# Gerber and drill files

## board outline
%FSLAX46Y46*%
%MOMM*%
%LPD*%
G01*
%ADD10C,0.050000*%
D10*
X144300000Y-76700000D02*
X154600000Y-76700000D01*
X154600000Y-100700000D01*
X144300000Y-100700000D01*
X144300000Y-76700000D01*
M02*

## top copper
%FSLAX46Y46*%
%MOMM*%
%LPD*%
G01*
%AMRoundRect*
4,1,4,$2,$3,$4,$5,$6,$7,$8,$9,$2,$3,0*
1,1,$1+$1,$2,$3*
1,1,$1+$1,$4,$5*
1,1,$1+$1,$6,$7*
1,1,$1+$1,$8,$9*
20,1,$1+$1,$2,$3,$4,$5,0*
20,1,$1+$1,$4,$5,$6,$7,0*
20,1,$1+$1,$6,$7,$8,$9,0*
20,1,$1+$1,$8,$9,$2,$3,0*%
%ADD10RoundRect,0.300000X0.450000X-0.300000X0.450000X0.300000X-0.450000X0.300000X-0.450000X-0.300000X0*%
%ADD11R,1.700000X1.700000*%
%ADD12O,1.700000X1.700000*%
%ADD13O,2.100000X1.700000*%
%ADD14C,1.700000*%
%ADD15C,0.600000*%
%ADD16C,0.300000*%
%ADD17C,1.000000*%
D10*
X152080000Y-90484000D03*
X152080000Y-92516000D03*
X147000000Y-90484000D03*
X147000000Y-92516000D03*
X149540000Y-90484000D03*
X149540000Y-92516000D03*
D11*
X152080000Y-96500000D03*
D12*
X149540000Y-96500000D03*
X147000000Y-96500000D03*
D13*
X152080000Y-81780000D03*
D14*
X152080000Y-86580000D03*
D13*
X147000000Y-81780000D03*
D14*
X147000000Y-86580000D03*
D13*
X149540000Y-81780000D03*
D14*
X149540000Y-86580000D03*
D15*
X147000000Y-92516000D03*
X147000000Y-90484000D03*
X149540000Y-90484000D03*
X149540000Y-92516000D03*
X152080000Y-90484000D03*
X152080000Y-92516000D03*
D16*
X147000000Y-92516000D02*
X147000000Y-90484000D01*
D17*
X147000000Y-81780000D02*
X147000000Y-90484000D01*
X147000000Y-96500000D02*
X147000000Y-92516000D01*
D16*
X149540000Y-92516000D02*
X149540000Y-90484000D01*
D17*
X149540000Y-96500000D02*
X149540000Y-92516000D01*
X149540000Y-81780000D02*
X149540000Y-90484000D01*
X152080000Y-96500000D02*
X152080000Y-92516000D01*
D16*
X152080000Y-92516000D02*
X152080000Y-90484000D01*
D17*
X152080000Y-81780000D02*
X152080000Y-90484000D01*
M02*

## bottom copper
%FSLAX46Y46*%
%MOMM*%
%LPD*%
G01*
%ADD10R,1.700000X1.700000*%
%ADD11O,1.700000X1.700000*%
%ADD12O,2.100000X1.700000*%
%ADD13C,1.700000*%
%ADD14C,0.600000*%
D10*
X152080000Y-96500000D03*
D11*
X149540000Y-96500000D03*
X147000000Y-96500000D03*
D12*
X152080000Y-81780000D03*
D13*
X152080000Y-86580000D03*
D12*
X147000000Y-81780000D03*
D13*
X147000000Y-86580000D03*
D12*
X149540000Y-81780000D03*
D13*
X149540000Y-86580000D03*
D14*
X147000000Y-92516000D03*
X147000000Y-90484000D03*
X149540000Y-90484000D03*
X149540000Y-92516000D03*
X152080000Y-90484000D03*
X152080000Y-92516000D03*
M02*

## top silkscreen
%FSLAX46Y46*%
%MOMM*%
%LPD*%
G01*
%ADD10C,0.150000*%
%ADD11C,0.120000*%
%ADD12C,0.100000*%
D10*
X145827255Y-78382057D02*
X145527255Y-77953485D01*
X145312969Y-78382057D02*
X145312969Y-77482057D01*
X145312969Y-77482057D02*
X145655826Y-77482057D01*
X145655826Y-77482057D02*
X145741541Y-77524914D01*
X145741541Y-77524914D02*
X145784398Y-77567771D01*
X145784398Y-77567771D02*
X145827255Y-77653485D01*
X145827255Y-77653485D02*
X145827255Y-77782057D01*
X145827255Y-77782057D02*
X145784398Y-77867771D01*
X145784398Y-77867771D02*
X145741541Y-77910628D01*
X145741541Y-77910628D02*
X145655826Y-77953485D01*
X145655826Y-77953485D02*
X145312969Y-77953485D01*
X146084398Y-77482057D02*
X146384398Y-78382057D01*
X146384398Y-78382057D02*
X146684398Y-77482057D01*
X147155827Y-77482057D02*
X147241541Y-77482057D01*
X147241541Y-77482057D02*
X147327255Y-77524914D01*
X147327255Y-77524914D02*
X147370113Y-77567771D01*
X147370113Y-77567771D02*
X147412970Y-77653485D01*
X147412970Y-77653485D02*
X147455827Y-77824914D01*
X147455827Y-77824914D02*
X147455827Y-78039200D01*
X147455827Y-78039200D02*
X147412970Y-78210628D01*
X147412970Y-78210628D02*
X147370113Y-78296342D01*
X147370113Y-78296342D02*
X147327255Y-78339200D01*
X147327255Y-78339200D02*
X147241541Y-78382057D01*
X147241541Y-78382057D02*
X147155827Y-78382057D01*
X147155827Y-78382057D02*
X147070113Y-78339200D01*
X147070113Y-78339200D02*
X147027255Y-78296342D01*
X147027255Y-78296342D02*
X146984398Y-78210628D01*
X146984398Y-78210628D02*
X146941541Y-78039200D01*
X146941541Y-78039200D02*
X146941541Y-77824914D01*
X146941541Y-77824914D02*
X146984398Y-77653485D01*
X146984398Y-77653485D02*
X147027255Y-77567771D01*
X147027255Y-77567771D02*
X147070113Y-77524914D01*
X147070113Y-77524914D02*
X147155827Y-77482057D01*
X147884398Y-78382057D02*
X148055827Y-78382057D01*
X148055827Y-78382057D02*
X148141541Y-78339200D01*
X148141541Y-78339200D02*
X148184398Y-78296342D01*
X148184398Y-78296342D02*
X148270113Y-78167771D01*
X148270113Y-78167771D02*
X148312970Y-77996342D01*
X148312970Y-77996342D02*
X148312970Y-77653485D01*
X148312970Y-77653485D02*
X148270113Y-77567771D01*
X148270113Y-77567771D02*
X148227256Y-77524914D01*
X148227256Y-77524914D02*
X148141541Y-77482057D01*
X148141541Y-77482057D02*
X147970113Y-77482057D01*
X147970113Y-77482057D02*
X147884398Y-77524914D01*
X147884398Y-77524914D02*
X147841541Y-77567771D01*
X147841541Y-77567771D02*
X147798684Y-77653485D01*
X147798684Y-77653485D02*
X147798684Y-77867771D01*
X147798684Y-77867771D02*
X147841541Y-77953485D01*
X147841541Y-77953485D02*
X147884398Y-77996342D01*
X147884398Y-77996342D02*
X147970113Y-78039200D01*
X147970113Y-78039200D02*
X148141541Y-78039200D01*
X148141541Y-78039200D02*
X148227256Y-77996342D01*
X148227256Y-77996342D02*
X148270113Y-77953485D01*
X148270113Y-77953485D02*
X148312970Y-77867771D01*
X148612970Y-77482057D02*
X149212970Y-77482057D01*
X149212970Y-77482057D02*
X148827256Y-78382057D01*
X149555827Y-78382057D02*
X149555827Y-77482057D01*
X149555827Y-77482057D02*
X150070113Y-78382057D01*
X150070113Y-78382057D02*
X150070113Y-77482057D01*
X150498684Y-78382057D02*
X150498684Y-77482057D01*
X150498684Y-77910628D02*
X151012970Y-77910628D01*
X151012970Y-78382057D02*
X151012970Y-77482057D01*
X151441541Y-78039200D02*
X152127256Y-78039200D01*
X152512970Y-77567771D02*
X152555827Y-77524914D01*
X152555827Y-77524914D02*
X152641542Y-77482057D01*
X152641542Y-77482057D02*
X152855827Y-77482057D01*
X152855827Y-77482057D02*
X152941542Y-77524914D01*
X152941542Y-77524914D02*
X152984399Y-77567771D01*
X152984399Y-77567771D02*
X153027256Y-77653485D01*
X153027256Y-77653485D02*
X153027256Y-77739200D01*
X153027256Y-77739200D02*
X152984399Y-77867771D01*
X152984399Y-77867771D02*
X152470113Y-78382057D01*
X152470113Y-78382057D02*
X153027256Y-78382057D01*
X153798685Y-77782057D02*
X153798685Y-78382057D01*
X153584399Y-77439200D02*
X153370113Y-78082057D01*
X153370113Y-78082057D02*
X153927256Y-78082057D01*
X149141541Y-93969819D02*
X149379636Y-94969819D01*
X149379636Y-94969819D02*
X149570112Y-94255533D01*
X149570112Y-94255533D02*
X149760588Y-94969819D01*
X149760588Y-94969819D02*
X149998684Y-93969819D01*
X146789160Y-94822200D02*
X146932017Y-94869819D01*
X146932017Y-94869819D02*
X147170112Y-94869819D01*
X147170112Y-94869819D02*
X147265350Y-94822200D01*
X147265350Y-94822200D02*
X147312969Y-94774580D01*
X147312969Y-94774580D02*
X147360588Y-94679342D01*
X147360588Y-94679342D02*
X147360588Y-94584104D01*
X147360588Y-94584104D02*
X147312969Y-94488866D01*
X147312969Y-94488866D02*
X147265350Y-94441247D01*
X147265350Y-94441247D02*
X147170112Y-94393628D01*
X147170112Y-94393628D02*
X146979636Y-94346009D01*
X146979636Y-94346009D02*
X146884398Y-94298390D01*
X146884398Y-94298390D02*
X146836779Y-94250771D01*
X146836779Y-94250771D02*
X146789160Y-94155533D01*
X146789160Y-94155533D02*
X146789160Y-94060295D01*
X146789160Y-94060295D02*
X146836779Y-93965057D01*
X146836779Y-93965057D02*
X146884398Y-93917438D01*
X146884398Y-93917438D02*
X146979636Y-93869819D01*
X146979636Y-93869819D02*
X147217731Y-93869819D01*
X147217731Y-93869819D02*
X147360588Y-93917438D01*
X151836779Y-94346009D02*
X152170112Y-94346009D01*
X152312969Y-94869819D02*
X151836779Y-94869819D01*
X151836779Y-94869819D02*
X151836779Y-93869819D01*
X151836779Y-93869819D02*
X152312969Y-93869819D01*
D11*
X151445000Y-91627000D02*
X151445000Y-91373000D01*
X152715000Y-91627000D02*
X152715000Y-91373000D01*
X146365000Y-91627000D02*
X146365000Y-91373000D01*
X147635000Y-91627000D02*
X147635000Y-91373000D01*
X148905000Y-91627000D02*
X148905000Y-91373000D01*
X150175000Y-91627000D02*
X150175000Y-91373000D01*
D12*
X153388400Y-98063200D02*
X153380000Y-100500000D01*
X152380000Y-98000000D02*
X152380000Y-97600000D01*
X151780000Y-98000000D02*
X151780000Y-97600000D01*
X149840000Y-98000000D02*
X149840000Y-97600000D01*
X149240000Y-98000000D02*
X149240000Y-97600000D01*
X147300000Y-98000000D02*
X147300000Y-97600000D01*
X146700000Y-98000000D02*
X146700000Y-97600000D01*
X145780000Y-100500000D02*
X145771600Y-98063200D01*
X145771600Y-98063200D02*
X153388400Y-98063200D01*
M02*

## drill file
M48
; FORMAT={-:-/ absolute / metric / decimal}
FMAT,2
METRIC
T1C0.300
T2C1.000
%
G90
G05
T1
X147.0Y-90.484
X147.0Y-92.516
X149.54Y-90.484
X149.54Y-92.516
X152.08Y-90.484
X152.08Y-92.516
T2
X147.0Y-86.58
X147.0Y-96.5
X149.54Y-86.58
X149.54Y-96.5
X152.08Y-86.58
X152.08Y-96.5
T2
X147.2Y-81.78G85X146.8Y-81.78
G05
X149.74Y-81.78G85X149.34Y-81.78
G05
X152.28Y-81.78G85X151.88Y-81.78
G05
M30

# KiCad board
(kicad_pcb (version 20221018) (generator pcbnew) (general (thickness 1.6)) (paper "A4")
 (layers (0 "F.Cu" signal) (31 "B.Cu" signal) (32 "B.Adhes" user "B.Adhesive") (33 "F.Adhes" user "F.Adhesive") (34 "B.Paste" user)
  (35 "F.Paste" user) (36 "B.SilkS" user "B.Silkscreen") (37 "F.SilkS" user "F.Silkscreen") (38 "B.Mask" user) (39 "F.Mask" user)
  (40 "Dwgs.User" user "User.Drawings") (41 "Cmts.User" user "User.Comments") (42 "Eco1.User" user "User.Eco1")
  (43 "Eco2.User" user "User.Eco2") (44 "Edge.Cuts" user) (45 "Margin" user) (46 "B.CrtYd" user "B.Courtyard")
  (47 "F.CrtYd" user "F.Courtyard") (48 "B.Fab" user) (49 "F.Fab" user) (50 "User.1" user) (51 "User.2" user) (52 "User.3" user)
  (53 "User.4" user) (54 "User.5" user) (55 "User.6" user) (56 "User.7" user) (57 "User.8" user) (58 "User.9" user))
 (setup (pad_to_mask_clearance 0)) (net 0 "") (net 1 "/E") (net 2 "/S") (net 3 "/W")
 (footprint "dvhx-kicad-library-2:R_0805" (layer "F.Cu") (at 152.08 91.5)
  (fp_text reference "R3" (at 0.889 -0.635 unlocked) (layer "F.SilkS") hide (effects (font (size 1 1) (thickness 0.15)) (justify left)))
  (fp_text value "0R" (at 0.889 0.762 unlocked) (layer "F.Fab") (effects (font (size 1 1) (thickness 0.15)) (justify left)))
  (fp_line (start -0.635 0.127) (end -0.635 -0.127) (stroke (width 0.12) (type solid)) (layer "F.SilkS"))
  (fp_line (start 0.635 0.127) (end 0.635 -0.127) (stroke (width 0.12) (type solid)) (layer "F.SilkS"))
  (pad "1" smd roundrect (at 0 -1.016 90) (size 1.2 1.5) (layers "F.Cu" "F.Paste" "F.Mask") (roundrect_rratio 0.25) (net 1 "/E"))
  (pad "2" smd roundrect (at 0 1.016 90) (size 1.2 1.5) (layers "F.Cu" "F.Paste" "F.Mask") (roundrect_rratio 0.25) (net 1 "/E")))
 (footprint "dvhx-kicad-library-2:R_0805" (layer "F.Cu") (at 147 91.5)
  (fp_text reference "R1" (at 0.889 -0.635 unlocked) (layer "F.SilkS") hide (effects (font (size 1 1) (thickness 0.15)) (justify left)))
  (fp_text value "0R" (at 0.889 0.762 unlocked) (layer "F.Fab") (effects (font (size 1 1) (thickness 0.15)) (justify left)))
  (fp_line (start -0.635 0.127) (end -0.635 -0.127) (stroke (width 0.12) (type solid)) (layer "F.SilkS"))
  (fp_line (start 0.635 0.127) (end 0.635 -0.127) (stroke (width 0.12) (type solid)) (layer "F.SilkS"))
  (pad "1" smd roundrect (at 0 -1.016 90) (size 1.2 1.5) (layers "F.Cu" "F.Paste" "F.Mask") (roundrect_rratio 0.25) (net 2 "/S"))
  (pad "2" smd roundrect (at 0 1.016 90) (size 1.2 1.5) (layers "F.Cu" "F.Paste" "F.Mask") (roundrect_rratio 0.25) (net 2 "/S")))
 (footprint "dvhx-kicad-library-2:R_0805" (layer "F.Cu") (at 149.54 91.5)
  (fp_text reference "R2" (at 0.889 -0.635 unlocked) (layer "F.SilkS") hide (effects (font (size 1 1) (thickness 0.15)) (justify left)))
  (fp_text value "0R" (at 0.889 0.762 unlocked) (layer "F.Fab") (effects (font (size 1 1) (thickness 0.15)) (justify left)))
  (fp_line (start -0.635 0.127) (end -0.635 -0.127) (stroke (width 0.12) (type solid)) (layer "F.SilkS"))
  (fp_line (start 0.635 0.127) (end 0.635 -0.127) (stroke (width 0.12) (type solid)) (layer "F.SilkS"))
  (pad "1" smd roundrect (at 0 -1.016 90) (size 1.2 1.5) (layers "F.Cu" "F.Paste" "F.Mask") (roundrect_rratio 0.25) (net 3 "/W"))
  (pad "2" smd roundrect (at 0 1.016 90) (size 1.2 1.5) (layers "F.Cu" "F.Paste" "F.Mask") (roundrect_rratio 0.25) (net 3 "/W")))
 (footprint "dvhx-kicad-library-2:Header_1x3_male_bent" (layer "F.Cu") (at 152.08 96.5 180)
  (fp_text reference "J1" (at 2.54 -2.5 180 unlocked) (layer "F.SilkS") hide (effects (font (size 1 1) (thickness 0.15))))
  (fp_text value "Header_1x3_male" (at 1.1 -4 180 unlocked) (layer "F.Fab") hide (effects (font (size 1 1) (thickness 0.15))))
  (fp_line (start -1.3084 -1.5632) (end -1.3 -4) (stroke (width 0.1) (type default)) (layer "F.SilkS"))
  (fp_line (start -0.3 -1.5) (end -0.3 -1.1) (stroke (width 0.1) (type default)) (layer "F.SilkS"))
  (fp_line (start 0.3 -1.5) (end 0.3 -1.1) (stroke (width 0.1) (type default)) (layer "F.SilkS"))
  (fp_line (start 2.24 -1.5) (end 2.24 -1.1) (stroke (width 0.1) (type default)) (layer "F.SilkS"))
  (fp_line (start 2.84 -1.5) (end 2.84 -1.1) (stroke (width 0.1) (type default)) (layer "F.SilkS"))
  (fp_line (start 4.78 -1.5) (end 4.78 -1.1) (stroke (width 0.1) (type default)) (layer "F.SilkS"))
  (fp_line (start 5.38 -1.5) (end 5.38 -1.1) (stroke (width 0.1) (type default)) (layer "F.SilkS"))
  (fp_line (start 6.3 -4) (end 6.3084 -1.5632) (stroke (width 0.1) (type default)) (layer "F.SilkS"))
  (fp_line (start 6.3084 -1.5632) (end -1.3084 -1.5632) (stroke (width 0.1) (type default)) (layer "F.SilkS"))
  (pad "1" thru_hole rect (at 0 0 270) (size 1.7 1.7) (drill 1) (layers "*.Cu" "*.Mask") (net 1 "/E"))
  (pad "2" thru_hole oval (at 2.54 0 270) (size 1.7 1.7) (drill 1) (layers "*.Cu" "*.Mask") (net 3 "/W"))
  (pad "3" thru_hole oval (at 5.08 0 270) (size 1.7 1.7) (drill 1) (layers "*.Cu" "*.Mask") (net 2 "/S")))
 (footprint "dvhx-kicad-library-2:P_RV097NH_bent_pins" (layer "B.Cu") (at 147 76.7 -90)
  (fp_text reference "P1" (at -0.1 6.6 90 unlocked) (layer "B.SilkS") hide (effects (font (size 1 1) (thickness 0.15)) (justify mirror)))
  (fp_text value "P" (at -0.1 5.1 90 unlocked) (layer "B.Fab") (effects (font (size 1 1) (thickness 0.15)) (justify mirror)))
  (pad "E" thru_hole oval (at 5.08 -5.08 270) (size 1.7 2.1) (drill oval 1 1.4) (layers "*.Cu" "*.Mask") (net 1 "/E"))
  (pad "E" thru_hole circle (at 9.88 -5.08 270) (size 1.7 1.7) (drill 1) (layers "*.Cu" "*.Mask") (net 1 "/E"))
  (pad "S" thru_hole oval (at 5.08 0 270) (size 1.7 2.1) (drill oval 1 1.4) (layers "*.Cu" "*.Mask") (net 2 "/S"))
  (pad "S" thru_hole circle (at 9.88 0 270) (size 1.7 1.7) (drill 1) (layers "*.Cu" "*.Mask") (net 2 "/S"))
  (pad "W" thru_hole oval (at 5.08 -2.54 270) (size 1.7 2.1) (drill oval 1 1.4) (layers "*.Cu" "*.Mask") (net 3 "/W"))
  (pad "W" thru_hole circle (at 9.88 -2.54 270) (size 1.7 1.7) (drill 1) (layers "*.Cu" "*.Mask") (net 3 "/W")))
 (gr_rect (start 144.3 76.7) (end 154.6 100.7) (stroke (width 0.05) (type default)) (fill none) (layer "Edge.Cuts"))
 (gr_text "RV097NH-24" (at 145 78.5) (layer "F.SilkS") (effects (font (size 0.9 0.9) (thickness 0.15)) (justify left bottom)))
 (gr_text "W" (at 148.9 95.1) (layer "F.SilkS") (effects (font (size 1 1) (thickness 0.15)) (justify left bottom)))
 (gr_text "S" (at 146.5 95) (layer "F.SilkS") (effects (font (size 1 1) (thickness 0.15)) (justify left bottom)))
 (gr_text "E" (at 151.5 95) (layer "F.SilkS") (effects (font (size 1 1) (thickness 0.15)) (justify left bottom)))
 (segment (start 147 92.516) (end 147 90.484) (width 0.3) (layer "F.Cu") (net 2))
 (segment (start 147 81.78) (end 147 90.484) (width 1) (layer "F.Cu") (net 2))
 (segment (start 147 96.5) (end 147 92.516) (width 1) (layer "F.Cu") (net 2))
 (via (at 147 92.516) (size 0.6) (drill 0.3) (layers "F.Cu" "B.Cu") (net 2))
 (via (at 147 90.484) (size 0.6) (drill 0.3) (layers "F.Cu" "B.Cu") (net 2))
 (segment (start 149.54 92.516) (end 149.54 90.484) (width 0.3) (layer "F.Cu") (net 3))
 (segment (start 149.54 96.5) (end 149.54 92.516) (width 1) (layer "F.Cu") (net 3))
 (segment (start 149.54 81.78) (end 149.54 90.484) (width 1) (layer "F.Cu") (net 3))
 (via (at 149.54 90.484) (size 0.6) (drill 0.3) (layers "F.Cu" "B.Cu") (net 3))
 (via (at 149.54 92.516) (size 0.6) (drill 0.3) (layers "F.Cu" "B.Cu") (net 3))
 (segment (start 152.08 96.5) (end 152.08 92.516) (width 1) (layer "F.Cu") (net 1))
 (segment (start 152.08 92.516) (end 152.08 90.484) (width 0.3) (layer "F.Cu") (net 1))
 (segment (start 152.08 81.78) (end 152.08 90.484) (width 1) (layer "F.Cu") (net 1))
 (via (at 152.08 90.484) (size 0.6) (drill 0.3) (layers "F.Cu" "B.Cu") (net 1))
 (via (at 152.08 92.516) (size 0.6) (drill 0.3) (layers "F.Cu" "B.Cu") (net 1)))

